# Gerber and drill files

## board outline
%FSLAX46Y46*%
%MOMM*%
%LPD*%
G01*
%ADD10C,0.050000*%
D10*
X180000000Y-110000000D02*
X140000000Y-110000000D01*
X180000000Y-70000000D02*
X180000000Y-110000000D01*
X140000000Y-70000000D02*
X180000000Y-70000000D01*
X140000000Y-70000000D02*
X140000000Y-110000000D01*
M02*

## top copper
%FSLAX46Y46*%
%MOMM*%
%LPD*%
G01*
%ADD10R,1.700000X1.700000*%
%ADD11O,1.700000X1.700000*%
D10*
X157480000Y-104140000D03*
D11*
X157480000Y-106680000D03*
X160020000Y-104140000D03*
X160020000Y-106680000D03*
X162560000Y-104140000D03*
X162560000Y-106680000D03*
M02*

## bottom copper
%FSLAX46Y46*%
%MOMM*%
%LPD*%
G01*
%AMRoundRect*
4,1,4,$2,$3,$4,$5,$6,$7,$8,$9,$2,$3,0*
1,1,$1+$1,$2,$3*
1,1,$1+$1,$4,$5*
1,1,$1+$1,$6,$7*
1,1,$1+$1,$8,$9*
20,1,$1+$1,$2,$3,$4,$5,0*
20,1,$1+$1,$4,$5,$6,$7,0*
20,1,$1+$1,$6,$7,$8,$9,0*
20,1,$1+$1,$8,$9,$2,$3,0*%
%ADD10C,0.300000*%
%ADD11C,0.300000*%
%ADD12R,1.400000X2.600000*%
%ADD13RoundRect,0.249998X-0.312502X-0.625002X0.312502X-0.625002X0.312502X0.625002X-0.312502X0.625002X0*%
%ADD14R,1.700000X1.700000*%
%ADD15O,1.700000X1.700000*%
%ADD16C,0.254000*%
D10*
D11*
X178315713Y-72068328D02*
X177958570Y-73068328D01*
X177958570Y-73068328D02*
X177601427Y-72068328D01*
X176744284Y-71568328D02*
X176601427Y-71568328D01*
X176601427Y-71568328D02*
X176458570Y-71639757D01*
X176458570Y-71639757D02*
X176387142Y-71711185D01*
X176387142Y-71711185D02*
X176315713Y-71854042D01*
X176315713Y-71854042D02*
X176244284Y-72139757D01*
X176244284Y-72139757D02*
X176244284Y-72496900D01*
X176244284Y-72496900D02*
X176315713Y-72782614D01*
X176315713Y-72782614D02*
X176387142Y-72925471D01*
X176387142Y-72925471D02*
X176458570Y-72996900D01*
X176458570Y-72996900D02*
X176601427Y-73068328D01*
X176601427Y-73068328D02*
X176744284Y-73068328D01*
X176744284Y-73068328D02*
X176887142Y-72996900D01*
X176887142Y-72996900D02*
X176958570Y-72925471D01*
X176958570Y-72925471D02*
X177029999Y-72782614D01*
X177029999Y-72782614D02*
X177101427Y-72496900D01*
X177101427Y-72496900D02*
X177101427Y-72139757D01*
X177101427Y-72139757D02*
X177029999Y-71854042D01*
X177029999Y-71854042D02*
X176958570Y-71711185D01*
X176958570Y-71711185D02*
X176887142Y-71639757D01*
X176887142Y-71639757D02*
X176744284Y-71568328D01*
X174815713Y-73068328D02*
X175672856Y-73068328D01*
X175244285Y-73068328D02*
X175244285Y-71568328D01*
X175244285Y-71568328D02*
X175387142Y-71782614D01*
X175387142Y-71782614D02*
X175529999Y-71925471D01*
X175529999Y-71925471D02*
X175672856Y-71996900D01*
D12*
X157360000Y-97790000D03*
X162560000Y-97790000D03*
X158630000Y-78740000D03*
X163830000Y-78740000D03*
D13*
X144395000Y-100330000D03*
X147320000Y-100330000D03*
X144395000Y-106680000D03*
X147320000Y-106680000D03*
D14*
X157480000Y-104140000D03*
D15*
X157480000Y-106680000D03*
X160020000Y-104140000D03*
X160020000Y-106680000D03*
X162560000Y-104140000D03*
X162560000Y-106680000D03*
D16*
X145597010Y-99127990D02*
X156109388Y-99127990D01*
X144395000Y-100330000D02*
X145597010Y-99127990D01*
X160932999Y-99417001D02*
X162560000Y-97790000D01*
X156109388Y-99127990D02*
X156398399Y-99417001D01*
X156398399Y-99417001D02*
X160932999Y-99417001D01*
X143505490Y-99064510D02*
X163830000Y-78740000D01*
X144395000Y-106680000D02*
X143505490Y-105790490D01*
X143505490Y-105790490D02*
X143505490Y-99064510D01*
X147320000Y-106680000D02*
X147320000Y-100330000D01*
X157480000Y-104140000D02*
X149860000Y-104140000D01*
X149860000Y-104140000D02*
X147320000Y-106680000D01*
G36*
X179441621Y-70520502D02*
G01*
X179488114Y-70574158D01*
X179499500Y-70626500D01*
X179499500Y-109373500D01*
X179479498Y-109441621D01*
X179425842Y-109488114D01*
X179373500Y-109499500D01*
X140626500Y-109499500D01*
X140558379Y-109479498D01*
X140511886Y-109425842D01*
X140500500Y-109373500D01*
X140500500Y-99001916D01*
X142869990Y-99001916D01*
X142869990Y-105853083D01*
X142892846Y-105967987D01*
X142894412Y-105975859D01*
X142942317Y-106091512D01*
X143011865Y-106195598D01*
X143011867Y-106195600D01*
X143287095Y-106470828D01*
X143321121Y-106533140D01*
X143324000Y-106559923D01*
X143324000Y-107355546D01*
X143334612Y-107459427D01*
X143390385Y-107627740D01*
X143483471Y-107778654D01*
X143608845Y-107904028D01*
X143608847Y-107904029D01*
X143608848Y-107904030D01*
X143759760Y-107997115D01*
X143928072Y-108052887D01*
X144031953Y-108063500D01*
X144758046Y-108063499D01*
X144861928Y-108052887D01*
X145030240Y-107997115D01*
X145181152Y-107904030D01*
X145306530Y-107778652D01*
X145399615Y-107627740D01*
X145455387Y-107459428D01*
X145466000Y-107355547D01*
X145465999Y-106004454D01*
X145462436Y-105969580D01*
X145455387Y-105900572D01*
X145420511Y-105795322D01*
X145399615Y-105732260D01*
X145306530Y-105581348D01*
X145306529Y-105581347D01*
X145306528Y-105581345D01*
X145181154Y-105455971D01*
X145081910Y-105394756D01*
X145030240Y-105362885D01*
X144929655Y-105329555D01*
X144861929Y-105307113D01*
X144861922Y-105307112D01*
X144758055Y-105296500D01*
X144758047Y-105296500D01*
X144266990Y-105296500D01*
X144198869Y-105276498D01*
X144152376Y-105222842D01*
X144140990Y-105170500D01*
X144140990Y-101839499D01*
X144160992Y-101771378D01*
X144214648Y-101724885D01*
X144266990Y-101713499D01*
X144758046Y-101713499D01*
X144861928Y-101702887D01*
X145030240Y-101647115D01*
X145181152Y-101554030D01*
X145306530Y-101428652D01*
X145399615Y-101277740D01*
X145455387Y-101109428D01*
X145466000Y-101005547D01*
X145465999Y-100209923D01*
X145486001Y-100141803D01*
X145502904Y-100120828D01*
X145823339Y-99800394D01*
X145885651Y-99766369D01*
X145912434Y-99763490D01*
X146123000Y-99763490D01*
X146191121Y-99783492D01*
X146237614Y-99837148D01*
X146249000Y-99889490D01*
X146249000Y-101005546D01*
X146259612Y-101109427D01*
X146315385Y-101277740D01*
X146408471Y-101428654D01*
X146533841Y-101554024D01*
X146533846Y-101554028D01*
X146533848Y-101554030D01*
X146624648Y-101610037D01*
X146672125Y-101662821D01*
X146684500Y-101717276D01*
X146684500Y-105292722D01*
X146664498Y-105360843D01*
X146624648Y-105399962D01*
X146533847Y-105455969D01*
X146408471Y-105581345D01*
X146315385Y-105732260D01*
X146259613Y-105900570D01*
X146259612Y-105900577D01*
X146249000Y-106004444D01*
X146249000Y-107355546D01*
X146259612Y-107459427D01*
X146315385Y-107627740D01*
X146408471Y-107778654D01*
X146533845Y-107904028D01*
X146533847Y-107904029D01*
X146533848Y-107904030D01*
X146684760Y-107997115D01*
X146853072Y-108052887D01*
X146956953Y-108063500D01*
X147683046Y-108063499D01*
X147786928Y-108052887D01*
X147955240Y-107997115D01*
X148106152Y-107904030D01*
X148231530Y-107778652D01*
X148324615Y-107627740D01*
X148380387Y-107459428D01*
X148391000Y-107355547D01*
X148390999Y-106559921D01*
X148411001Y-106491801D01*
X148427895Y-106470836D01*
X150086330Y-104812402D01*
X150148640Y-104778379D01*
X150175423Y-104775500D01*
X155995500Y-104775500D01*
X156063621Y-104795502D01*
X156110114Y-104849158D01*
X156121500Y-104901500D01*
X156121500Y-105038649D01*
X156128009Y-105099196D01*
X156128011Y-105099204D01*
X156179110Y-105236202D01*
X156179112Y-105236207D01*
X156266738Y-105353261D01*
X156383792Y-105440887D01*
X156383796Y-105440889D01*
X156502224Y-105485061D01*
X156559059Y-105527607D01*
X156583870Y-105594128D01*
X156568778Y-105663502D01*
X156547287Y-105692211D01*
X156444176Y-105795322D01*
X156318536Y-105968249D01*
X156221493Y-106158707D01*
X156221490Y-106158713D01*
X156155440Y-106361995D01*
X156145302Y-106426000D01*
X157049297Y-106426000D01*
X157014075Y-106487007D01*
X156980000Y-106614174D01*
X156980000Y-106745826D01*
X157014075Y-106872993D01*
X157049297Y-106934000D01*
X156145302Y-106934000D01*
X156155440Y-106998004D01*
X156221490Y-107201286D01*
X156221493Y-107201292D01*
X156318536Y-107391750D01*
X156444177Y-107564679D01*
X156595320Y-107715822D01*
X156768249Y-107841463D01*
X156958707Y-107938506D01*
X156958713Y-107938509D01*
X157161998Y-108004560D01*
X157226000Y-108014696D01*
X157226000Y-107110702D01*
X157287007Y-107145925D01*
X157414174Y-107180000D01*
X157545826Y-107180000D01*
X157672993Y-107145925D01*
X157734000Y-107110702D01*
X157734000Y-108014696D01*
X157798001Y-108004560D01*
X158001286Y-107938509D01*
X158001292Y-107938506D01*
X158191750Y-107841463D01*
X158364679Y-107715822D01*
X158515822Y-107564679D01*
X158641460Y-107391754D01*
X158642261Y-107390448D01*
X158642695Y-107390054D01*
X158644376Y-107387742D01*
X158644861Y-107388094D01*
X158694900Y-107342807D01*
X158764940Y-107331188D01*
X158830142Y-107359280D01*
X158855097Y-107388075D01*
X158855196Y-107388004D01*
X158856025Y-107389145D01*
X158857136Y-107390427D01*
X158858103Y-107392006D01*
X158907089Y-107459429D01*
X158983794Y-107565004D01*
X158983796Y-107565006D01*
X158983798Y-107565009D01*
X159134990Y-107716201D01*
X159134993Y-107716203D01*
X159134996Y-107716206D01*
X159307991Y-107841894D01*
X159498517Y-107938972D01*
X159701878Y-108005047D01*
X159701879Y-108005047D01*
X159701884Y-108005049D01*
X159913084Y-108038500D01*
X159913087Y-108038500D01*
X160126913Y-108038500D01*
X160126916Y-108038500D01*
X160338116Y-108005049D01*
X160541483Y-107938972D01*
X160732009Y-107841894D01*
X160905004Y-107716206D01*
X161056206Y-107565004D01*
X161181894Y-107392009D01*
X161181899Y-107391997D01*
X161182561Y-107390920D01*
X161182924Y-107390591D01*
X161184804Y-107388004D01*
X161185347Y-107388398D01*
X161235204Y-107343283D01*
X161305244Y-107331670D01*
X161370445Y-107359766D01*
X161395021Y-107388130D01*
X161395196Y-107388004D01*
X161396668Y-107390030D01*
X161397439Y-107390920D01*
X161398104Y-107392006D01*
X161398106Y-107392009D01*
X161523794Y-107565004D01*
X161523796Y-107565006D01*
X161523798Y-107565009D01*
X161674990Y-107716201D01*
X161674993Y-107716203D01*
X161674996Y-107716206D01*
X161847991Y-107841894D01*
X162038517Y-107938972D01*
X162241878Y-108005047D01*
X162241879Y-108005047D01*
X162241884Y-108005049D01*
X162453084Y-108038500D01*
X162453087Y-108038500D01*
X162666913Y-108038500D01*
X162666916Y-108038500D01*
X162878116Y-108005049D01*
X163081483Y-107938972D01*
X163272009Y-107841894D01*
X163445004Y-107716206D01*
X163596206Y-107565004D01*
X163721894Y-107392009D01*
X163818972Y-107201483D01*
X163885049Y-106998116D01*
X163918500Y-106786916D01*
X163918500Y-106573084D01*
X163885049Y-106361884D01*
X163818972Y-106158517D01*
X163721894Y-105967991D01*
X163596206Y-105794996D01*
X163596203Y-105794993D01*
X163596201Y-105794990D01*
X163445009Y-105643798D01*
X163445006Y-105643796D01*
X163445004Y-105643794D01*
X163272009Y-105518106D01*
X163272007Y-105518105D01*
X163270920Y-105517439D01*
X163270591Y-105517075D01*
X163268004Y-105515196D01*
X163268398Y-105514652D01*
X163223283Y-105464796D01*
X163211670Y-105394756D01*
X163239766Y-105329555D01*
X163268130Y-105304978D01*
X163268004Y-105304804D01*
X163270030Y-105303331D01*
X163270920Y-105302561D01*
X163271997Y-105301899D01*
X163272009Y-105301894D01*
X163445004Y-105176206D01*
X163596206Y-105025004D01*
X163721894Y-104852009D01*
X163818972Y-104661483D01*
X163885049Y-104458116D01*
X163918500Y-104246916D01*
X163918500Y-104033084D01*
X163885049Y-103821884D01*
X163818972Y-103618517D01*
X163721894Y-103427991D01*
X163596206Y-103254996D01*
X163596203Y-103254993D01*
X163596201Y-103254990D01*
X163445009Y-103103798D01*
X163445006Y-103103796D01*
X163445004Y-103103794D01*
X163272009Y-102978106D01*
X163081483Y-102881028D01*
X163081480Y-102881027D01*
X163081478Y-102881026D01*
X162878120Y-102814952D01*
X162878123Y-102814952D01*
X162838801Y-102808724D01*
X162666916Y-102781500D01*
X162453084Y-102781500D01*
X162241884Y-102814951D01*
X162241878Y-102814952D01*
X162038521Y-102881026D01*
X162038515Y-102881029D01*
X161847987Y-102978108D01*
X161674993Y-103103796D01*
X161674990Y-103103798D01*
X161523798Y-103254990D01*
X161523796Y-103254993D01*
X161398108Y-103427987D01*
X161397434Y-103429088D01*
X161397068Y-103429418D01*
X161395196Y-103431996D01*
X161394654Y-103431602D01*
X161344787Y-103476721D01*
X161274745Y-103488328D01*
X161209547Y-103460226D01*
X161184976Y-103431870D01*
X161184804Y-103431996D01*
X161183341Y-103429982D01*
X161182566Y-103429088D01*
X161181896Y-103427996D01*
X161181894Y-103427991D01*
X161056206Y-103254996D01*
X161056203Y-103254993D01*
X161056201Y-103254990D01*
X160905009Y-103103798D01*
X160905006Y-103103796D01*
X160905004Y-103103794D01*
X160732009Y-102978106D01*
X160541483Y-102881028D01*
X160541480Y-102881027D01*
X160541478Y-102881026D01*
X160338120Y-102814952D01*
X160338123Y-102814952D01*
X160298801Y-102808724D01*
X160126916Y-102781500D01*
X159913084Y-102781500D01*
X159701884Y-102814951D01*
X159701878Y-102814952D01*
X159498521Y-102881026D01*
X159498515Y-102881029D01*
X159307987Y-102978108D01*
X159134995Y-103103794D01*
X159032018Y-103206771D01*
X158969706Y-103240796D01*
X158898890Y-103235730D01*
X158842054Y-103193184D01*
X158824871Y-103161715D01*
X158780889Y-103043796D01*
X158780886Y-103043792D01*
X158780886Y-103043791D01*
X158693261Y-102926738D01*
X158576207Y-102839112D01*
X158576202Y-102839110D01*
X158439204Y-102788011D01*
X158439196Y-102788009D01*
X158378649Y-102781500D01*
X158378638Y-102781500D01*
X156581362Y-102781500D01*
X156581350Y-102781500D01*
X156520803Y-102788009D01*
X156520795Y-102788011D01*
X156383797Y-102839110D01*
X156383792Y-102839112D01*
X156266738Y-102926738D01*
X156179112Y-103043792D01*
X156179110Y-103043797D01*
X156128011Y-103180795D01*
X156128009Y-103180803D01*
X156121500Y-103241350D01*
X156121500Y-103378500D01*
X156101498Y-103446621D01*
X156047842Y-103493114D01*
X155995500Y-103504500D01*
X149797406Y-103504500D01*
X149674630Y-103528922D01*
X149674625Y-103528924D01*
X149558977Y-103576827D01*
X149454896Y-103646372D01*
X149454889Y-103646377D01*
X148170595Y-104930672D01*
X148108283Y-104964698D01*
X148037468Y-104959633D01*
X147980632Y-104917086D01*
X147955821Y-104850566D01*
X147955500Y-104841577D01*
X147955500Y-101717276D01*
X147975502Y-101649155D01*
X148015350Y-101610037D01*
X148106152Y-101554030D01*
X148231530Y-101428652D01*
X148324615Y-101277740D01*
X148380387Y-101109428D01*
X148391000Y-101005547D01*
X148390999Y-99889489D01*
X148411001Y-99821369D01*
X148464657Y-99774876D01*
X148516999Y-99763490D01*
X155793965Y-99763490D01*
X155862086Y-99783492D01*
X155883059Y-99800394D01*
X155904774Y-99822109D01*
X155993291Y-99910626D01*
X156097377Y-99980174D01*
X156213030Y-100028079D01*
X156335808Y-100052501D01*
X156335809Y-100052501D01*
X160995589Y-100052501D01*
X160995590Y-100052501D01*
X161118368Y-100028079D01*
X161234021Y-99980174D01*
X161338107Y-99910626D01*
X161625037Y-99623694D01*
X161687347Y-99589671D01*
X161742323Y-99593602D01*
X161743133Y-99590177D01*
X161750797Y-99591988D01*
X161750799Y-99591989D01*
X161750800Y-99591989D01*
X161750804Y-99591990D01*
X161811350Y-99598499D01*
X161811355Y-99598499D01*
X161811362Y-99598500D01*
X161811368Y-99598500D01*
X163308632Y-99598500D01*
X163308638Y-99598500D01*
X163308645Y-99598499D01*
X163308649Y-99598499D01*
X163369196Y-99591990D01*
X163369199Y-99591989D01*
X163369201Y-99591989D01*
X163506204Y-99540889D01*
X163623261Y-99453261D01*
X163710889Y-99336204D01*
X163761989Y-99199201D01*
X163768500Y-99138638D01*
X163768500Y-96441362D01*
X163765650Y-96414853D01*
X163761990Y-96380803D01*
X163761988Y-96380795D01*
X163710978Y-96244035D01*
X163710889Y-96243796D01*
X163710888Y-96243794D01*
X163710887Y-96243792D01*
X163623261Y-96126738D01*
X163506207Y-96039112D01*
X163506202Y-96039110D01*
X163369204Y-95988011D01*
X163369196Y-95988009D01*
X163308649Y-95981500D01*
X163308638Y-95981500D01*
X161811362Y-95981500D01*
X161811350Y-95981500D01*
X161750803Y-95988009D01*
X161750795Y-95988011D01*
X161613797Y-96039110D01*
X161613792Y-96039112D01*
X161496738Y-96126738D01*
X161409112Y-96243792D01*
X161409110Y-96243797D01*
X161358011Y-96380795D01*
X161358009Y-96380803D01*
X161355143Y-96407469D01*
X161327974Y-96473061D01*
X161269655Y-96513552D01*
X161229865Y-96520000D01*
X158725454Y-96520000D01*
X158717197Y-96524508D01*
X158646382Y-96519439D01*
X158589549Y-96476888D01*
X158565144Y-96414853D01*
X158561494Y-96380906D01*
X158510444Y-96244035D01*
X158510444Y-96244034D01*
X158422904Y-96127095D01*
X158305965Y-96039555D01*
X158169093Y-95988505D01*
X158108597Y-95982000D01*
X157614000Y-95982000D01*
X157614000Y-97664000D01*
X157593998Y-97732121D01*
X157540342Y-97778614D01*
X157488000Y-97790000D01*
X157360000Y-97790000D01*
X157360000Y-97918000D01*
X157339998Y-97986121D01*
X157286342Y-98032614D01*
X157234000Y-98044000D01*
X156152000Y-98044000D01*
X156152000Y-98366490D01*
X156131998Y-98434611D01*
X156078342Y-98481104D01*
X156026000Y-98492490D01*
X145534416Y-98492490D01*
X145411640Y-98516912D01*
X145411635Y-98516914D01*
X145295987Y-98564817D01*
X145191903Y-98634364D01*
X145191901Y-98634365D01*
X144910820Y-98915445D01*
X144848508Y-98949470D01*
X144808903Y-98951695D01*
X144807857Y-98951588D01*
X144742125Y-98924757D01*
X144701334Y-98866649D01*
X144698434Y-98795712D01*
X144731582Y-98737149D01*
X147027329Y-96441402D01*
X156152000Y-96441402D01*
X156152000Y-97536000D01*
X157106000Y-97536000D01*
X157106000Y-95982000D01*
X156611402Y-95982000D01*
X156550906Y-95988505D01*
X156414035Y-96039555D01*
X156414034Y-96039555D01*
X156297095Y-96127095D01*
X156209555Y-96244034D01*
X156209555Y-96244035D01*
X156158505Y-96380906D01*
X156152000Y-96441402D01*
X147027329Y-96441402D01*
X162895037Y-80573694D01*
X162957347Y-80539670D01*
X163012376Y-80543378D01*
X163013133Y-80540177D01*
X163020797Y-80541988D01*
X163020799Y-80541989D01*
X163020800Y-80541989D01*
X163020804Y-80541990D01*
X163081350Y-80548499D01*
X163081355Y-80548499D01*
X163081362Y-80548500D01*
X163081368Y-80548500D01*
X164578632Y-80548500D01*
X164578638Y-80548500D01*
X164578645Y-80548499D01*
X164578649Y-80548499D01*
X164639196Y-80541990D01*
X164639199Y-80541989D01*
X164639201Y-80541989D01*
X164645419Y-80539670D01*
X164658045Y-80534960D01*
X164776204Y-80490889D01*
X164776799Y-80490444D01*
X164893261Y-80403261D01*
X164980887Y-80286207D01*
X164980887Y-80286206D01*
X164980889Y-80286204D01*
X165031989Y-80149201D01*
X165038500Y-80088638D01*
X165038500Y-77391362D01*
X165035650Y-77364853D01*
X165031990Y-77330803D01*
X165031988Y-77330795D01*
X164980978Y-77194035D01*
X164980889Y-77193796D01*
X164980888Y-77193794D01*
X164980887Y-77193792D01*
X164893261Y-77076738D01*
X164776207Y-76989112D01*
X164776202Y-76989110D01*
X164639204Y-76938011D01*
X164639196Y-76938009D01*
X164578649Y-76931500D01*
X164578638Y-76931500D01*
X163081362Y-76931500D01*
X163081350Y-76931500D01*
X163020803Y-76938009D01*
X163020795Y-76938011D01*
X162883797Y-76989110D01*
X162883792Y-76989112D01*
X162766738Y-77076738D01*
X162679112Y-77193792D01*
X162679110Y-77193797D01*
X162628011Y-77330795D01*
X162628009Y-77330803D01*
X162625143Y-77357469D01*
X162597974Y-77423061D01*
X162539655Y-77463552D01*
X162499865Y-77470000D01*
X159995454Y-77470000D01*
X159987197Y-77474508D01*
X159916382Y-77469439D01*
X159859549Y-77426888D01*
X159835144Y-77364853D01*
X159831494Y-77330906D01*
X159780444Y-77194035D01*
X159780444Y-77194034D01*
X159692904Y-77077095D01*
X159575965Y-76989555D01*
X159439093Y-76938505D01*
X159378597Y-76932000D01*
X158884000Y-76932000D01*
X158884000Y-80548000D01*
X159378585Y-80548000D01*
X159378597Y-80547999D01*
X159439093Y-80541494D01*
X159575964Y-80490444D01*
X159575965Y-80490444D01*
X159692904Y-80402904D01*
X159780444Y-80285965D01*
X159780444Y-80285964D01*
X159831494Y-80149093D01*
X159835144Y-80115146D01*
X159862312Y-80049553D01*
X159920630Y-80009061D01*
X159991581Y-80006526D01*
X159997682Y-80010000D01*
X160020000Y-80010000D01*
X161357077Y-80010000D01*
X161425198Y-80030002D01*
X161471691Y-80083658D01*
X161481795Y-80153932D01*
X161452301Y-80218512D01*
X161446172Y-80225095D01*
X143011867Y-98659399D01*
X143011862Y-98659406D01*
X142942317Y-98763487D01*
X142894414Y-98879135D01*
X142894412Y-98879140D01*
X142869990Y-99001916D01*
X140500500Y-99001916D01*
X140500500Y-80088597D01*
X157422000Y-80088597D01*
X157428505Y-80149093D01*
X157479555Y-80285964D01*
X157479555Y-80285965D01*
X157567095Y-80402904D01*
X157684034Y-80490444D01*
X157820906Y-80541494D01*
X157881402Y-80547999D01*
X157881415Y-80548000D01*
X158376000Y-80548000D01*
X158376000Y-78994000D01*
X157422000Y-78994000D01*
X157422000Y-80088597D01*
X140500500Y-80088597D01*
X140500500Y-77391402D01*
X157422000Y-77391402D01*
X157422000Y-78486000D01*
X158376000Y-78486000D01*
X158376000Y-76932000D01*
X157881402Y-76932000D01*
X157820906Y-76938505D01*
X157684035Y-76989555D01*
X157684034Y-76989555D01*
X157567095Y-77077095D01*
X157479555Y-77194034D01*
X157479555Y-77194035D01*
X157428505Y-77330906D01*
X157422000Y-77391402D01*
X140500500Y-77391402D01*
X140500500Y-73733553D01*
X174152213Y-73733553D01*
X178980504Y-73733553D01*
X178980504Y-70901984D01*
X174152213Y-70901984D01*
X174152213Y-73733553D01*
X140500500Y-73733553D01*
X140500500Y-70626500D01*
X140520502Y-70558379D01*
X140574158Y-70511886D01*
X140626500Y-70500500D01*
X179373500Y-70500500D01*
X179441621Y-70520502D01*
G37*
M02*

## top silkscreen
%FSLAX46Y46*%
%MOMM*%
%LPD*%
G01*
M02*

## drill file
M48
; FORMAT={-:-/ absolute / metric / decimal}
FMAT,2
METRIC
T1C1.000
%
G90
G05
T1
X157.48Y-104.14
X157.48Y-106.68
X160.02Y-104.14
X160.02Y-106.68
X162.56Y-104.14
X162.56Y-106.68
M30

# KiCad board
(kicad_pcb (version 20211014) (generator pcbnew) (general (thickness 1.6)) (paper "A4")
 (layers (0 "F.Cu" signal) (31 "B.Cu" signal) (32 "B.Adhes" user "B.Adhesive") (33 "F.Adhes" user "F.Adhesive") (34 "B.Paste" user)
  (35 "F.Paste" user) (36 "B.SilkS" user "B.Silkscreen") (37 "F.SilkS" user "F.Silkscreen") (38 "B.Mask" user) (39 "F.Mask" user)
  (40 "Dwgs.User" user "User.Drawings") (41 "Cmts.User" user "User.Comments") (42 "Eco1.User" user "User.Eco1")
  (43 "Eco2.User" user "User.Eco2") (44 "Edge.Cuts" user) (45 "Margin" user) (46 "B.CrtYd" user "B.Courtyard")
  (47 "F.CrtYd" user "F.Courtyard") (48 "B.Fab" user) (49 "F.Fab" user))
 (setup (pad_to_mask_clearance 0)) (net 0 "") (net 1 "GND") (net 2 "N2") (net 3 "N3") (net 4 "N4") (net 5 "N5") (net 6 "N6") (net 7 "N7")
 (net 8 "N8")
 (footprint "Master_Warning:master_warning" (layer "F.Cu") (at 160.728956 89.510401)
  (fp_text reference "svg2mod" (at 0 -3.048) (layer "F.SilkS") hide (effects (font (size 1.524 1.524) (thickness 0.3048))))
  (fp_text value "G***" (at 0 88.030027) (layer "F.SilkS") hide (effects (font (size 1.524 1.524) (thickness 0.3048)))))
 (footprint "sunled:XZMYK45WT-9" (layer "B.Cu") (at 159.96 97.79)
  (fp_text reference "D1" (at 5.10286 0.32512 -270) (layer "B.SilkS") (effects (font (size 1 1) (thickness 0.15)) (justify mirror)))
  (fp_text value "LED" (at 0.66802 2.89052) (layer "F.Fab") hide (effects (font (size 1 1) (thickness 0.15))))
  (pad "1" smd rect locked (at -2.6 0) (size 1.4 2.6) (layers "B.Cu" "B.Paste" "B.Mask") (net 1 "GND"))
  (pad "2" smd rect locked (at 2.6 0) (size 1.4 2.6) (layers "B.Cu" "B.Paste" "B.Mask") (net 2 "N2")))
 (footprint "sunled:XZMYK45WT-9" (layer "B.Cu") (at 161.23 78.74)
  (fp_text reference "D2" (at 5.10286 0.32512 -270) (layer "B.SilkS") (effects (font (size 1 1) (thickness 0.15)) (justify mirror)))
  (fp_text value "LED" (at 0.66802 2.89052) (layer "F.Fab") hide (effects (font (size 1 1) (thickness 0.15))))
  (pad "1" smd rect locked (at -2.6 0) (size 1.4 2.6) (layers "B.Cu" "B.Paste" "B.Mask") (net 1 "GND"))
  (pad "2" smd rect locked (at 2.6 0) (size 1.4 2.6) (layers "B.Cu" "B.Paste" "B.Mask") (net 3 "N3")))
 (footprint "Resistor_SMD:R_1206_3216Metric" (layer "B.Cu") (at 145.8575 100.33)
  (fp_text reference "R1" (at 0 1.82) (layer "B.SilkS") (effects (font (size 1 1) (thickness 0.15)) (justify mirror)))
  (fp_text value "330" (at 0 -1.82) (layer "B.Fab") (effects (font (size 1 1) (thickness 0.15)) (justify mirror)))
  (pad "1" smd roundrect locked (at -1.4625 0) (size 1.125 1.75) (layers "B.Cu" "B.Paste" "B.Mask") (roundrect_rratio 0.2222204444)
   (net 2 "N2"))
  (pad "2" smd roundrect locked (at 1.4625 0) (size 1.125 1.75) (layers "B.Cu" "B.Paste" "B.Mask") (roundrect_rratio 0.2222204444)
   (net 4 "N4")))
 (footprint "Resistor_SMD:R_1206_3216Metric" (layer "B.Cu") (at 145.8575 106.68)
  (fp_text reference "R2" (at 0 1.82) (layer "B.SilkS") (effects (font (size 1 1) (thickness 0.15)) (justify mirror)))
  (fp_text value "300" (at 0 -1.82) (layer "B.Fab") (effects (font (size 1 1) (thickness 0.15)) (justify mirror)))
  (pad "1" smd roundrect locked (at -1.4625 0) (size 1.125 1.75) (layers "B.Cu" "B.Paste" "B.Mask") (roundrect_rratio 0.2222204444)
   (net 3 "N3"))
  (pad "2" smd roundrect locked (at 1.4625 0) (size 1.125 1.75) (layers "B.Cu" "B.Paste" "B.Mask") (roundrect_rratio 0.2222204444)
   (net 4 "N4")))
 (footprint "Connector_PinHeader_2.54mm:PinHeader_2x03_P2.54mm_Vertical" (layer "B.Cu") (at 157.48 104.14 -90)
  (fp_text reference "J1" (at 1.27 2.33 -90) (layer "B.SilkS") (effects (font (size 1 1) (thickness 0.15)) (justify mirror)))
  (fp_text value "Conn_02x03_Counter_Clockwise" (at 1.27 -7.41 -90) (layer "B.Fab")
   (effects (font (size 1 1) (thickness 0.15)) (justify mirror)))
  (pad "1" thru_hole rect locked (at 0 0 270) (size 1.7 1.7) (drill 1) (layers *.Cu *.Mask) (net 4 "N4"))
  (pad "2" thru_hole oval locked (at 2.54 0 270) (size 1.7 1.7) (drill 1) (layers *.Cu *.Mask) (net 1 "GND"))
  (pad "3" thru_hole oval locked (at 0 -2.54 270) (size 1.7 1.7) (drill 1) (layers *.Cu *.Mask) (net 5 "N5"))
  (pad "4" thru_hole oval locked (at 2.54 -2.54 270) (size 1.7 1.7) (drill 1) (layers *.Cu *.Mask) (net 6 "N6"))
  (pad "5" thru_hole oval locked (at 0 -5.08 270) (size 1.7 1.7) (drill 1) (layers *.Cu *.Mask) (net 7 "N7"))
  (pad "6" thru_hole oval locked (at 2.54 -5.08 270) (size 1.7 1.7) (drill 1) (layers *.Cu *.Mask) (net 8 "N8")))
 (gr_line (start 180 110) (end 140 110) (layer "Edge.Cuts") (width 0.05))
 (gr_line (start 180 70) (end 180 110) (layer "Edge.Cuts") (width 0.05))
 (gr_line (start 140 70) (end 180 70) (layer "Edge.Cuts") (width 0.05))
 (gr_line (start 140 70) (end 140 110) (layer "Edge.Cuts") (width 0.05))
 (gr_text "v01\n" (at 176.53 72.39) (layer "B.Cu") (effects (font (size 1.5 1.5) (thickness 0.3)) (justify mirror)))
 (segment (start 145.59701 99.12799) (end 156.109388 99.12799) (width 0.254) (layer "B.Cu") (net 2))
 (segment (start 144.395 100.33) (end 145.59701 99.12799) (width 0.254) (layer "B.Cu") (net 2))
 (segment (start 160.932999 99.417001) (end 162.56 97.79) (width 0.254) (layer "B.Cu") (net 2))
 (segment (start 156.109388 99.12799) (end 156.398399 99.417001) (width 0.254) (layer "B.Cu") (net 2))
 (segment (start 156.398399 99.417001) (end 160.932999 99.417001) (width 0.254) (layer "B.Cu") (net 2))
 (segment (start 143.50549 99.06451) (end 163.83 78.74) (width 0.254) (layer "B.Cu") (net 3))
 (segment (start 144.395 106.68) (end 143.50549 105.79049) (width 0.254) (layer "B.Cu") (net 3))
 (segment (start 143.50549 105.79049) (end 143.50549 99.06451) (width 0.254) (layer "B.Cu") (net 3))
 (segment (start 147.32 106.68) (end 147.32 100.33) (width 0.254) (layer "B.Cu") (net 4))
 (segment (start 157.48 104.14) (end 149.86 104.14) (width 0.254) (layer "B.Cu") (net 4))
 (segment (start 149.86 104.14) (end 147.32 106.68) (width 0.254) (layer "B.Cu") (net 4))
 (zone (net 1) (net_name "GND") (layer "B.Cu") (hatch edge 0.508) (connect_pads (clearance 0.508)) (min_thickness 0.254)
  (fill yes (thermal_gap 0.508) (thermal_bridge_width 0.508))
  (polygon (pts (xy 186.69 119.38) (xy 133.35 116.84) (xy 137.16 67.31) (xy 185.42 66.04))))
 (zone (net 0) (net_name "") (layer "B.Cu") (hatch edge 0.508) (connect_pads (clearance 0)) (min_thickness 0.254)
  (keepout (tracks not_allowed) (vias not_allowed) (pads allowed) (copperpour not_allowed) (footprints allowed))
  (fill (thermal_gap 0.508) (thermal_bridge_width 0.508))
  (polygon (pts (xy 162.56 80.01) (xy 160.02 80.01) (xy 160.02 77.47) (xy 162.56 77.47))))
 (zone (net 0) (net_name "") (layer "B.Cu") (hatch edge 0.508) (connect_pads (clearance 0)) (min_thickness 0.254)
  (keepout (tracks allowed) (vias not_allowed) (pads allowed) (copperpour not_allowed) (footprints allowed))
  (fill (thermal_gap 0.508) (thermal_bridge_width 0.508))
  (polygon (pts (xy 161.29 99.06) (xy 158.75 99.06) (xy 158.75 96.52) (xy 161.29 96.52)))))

